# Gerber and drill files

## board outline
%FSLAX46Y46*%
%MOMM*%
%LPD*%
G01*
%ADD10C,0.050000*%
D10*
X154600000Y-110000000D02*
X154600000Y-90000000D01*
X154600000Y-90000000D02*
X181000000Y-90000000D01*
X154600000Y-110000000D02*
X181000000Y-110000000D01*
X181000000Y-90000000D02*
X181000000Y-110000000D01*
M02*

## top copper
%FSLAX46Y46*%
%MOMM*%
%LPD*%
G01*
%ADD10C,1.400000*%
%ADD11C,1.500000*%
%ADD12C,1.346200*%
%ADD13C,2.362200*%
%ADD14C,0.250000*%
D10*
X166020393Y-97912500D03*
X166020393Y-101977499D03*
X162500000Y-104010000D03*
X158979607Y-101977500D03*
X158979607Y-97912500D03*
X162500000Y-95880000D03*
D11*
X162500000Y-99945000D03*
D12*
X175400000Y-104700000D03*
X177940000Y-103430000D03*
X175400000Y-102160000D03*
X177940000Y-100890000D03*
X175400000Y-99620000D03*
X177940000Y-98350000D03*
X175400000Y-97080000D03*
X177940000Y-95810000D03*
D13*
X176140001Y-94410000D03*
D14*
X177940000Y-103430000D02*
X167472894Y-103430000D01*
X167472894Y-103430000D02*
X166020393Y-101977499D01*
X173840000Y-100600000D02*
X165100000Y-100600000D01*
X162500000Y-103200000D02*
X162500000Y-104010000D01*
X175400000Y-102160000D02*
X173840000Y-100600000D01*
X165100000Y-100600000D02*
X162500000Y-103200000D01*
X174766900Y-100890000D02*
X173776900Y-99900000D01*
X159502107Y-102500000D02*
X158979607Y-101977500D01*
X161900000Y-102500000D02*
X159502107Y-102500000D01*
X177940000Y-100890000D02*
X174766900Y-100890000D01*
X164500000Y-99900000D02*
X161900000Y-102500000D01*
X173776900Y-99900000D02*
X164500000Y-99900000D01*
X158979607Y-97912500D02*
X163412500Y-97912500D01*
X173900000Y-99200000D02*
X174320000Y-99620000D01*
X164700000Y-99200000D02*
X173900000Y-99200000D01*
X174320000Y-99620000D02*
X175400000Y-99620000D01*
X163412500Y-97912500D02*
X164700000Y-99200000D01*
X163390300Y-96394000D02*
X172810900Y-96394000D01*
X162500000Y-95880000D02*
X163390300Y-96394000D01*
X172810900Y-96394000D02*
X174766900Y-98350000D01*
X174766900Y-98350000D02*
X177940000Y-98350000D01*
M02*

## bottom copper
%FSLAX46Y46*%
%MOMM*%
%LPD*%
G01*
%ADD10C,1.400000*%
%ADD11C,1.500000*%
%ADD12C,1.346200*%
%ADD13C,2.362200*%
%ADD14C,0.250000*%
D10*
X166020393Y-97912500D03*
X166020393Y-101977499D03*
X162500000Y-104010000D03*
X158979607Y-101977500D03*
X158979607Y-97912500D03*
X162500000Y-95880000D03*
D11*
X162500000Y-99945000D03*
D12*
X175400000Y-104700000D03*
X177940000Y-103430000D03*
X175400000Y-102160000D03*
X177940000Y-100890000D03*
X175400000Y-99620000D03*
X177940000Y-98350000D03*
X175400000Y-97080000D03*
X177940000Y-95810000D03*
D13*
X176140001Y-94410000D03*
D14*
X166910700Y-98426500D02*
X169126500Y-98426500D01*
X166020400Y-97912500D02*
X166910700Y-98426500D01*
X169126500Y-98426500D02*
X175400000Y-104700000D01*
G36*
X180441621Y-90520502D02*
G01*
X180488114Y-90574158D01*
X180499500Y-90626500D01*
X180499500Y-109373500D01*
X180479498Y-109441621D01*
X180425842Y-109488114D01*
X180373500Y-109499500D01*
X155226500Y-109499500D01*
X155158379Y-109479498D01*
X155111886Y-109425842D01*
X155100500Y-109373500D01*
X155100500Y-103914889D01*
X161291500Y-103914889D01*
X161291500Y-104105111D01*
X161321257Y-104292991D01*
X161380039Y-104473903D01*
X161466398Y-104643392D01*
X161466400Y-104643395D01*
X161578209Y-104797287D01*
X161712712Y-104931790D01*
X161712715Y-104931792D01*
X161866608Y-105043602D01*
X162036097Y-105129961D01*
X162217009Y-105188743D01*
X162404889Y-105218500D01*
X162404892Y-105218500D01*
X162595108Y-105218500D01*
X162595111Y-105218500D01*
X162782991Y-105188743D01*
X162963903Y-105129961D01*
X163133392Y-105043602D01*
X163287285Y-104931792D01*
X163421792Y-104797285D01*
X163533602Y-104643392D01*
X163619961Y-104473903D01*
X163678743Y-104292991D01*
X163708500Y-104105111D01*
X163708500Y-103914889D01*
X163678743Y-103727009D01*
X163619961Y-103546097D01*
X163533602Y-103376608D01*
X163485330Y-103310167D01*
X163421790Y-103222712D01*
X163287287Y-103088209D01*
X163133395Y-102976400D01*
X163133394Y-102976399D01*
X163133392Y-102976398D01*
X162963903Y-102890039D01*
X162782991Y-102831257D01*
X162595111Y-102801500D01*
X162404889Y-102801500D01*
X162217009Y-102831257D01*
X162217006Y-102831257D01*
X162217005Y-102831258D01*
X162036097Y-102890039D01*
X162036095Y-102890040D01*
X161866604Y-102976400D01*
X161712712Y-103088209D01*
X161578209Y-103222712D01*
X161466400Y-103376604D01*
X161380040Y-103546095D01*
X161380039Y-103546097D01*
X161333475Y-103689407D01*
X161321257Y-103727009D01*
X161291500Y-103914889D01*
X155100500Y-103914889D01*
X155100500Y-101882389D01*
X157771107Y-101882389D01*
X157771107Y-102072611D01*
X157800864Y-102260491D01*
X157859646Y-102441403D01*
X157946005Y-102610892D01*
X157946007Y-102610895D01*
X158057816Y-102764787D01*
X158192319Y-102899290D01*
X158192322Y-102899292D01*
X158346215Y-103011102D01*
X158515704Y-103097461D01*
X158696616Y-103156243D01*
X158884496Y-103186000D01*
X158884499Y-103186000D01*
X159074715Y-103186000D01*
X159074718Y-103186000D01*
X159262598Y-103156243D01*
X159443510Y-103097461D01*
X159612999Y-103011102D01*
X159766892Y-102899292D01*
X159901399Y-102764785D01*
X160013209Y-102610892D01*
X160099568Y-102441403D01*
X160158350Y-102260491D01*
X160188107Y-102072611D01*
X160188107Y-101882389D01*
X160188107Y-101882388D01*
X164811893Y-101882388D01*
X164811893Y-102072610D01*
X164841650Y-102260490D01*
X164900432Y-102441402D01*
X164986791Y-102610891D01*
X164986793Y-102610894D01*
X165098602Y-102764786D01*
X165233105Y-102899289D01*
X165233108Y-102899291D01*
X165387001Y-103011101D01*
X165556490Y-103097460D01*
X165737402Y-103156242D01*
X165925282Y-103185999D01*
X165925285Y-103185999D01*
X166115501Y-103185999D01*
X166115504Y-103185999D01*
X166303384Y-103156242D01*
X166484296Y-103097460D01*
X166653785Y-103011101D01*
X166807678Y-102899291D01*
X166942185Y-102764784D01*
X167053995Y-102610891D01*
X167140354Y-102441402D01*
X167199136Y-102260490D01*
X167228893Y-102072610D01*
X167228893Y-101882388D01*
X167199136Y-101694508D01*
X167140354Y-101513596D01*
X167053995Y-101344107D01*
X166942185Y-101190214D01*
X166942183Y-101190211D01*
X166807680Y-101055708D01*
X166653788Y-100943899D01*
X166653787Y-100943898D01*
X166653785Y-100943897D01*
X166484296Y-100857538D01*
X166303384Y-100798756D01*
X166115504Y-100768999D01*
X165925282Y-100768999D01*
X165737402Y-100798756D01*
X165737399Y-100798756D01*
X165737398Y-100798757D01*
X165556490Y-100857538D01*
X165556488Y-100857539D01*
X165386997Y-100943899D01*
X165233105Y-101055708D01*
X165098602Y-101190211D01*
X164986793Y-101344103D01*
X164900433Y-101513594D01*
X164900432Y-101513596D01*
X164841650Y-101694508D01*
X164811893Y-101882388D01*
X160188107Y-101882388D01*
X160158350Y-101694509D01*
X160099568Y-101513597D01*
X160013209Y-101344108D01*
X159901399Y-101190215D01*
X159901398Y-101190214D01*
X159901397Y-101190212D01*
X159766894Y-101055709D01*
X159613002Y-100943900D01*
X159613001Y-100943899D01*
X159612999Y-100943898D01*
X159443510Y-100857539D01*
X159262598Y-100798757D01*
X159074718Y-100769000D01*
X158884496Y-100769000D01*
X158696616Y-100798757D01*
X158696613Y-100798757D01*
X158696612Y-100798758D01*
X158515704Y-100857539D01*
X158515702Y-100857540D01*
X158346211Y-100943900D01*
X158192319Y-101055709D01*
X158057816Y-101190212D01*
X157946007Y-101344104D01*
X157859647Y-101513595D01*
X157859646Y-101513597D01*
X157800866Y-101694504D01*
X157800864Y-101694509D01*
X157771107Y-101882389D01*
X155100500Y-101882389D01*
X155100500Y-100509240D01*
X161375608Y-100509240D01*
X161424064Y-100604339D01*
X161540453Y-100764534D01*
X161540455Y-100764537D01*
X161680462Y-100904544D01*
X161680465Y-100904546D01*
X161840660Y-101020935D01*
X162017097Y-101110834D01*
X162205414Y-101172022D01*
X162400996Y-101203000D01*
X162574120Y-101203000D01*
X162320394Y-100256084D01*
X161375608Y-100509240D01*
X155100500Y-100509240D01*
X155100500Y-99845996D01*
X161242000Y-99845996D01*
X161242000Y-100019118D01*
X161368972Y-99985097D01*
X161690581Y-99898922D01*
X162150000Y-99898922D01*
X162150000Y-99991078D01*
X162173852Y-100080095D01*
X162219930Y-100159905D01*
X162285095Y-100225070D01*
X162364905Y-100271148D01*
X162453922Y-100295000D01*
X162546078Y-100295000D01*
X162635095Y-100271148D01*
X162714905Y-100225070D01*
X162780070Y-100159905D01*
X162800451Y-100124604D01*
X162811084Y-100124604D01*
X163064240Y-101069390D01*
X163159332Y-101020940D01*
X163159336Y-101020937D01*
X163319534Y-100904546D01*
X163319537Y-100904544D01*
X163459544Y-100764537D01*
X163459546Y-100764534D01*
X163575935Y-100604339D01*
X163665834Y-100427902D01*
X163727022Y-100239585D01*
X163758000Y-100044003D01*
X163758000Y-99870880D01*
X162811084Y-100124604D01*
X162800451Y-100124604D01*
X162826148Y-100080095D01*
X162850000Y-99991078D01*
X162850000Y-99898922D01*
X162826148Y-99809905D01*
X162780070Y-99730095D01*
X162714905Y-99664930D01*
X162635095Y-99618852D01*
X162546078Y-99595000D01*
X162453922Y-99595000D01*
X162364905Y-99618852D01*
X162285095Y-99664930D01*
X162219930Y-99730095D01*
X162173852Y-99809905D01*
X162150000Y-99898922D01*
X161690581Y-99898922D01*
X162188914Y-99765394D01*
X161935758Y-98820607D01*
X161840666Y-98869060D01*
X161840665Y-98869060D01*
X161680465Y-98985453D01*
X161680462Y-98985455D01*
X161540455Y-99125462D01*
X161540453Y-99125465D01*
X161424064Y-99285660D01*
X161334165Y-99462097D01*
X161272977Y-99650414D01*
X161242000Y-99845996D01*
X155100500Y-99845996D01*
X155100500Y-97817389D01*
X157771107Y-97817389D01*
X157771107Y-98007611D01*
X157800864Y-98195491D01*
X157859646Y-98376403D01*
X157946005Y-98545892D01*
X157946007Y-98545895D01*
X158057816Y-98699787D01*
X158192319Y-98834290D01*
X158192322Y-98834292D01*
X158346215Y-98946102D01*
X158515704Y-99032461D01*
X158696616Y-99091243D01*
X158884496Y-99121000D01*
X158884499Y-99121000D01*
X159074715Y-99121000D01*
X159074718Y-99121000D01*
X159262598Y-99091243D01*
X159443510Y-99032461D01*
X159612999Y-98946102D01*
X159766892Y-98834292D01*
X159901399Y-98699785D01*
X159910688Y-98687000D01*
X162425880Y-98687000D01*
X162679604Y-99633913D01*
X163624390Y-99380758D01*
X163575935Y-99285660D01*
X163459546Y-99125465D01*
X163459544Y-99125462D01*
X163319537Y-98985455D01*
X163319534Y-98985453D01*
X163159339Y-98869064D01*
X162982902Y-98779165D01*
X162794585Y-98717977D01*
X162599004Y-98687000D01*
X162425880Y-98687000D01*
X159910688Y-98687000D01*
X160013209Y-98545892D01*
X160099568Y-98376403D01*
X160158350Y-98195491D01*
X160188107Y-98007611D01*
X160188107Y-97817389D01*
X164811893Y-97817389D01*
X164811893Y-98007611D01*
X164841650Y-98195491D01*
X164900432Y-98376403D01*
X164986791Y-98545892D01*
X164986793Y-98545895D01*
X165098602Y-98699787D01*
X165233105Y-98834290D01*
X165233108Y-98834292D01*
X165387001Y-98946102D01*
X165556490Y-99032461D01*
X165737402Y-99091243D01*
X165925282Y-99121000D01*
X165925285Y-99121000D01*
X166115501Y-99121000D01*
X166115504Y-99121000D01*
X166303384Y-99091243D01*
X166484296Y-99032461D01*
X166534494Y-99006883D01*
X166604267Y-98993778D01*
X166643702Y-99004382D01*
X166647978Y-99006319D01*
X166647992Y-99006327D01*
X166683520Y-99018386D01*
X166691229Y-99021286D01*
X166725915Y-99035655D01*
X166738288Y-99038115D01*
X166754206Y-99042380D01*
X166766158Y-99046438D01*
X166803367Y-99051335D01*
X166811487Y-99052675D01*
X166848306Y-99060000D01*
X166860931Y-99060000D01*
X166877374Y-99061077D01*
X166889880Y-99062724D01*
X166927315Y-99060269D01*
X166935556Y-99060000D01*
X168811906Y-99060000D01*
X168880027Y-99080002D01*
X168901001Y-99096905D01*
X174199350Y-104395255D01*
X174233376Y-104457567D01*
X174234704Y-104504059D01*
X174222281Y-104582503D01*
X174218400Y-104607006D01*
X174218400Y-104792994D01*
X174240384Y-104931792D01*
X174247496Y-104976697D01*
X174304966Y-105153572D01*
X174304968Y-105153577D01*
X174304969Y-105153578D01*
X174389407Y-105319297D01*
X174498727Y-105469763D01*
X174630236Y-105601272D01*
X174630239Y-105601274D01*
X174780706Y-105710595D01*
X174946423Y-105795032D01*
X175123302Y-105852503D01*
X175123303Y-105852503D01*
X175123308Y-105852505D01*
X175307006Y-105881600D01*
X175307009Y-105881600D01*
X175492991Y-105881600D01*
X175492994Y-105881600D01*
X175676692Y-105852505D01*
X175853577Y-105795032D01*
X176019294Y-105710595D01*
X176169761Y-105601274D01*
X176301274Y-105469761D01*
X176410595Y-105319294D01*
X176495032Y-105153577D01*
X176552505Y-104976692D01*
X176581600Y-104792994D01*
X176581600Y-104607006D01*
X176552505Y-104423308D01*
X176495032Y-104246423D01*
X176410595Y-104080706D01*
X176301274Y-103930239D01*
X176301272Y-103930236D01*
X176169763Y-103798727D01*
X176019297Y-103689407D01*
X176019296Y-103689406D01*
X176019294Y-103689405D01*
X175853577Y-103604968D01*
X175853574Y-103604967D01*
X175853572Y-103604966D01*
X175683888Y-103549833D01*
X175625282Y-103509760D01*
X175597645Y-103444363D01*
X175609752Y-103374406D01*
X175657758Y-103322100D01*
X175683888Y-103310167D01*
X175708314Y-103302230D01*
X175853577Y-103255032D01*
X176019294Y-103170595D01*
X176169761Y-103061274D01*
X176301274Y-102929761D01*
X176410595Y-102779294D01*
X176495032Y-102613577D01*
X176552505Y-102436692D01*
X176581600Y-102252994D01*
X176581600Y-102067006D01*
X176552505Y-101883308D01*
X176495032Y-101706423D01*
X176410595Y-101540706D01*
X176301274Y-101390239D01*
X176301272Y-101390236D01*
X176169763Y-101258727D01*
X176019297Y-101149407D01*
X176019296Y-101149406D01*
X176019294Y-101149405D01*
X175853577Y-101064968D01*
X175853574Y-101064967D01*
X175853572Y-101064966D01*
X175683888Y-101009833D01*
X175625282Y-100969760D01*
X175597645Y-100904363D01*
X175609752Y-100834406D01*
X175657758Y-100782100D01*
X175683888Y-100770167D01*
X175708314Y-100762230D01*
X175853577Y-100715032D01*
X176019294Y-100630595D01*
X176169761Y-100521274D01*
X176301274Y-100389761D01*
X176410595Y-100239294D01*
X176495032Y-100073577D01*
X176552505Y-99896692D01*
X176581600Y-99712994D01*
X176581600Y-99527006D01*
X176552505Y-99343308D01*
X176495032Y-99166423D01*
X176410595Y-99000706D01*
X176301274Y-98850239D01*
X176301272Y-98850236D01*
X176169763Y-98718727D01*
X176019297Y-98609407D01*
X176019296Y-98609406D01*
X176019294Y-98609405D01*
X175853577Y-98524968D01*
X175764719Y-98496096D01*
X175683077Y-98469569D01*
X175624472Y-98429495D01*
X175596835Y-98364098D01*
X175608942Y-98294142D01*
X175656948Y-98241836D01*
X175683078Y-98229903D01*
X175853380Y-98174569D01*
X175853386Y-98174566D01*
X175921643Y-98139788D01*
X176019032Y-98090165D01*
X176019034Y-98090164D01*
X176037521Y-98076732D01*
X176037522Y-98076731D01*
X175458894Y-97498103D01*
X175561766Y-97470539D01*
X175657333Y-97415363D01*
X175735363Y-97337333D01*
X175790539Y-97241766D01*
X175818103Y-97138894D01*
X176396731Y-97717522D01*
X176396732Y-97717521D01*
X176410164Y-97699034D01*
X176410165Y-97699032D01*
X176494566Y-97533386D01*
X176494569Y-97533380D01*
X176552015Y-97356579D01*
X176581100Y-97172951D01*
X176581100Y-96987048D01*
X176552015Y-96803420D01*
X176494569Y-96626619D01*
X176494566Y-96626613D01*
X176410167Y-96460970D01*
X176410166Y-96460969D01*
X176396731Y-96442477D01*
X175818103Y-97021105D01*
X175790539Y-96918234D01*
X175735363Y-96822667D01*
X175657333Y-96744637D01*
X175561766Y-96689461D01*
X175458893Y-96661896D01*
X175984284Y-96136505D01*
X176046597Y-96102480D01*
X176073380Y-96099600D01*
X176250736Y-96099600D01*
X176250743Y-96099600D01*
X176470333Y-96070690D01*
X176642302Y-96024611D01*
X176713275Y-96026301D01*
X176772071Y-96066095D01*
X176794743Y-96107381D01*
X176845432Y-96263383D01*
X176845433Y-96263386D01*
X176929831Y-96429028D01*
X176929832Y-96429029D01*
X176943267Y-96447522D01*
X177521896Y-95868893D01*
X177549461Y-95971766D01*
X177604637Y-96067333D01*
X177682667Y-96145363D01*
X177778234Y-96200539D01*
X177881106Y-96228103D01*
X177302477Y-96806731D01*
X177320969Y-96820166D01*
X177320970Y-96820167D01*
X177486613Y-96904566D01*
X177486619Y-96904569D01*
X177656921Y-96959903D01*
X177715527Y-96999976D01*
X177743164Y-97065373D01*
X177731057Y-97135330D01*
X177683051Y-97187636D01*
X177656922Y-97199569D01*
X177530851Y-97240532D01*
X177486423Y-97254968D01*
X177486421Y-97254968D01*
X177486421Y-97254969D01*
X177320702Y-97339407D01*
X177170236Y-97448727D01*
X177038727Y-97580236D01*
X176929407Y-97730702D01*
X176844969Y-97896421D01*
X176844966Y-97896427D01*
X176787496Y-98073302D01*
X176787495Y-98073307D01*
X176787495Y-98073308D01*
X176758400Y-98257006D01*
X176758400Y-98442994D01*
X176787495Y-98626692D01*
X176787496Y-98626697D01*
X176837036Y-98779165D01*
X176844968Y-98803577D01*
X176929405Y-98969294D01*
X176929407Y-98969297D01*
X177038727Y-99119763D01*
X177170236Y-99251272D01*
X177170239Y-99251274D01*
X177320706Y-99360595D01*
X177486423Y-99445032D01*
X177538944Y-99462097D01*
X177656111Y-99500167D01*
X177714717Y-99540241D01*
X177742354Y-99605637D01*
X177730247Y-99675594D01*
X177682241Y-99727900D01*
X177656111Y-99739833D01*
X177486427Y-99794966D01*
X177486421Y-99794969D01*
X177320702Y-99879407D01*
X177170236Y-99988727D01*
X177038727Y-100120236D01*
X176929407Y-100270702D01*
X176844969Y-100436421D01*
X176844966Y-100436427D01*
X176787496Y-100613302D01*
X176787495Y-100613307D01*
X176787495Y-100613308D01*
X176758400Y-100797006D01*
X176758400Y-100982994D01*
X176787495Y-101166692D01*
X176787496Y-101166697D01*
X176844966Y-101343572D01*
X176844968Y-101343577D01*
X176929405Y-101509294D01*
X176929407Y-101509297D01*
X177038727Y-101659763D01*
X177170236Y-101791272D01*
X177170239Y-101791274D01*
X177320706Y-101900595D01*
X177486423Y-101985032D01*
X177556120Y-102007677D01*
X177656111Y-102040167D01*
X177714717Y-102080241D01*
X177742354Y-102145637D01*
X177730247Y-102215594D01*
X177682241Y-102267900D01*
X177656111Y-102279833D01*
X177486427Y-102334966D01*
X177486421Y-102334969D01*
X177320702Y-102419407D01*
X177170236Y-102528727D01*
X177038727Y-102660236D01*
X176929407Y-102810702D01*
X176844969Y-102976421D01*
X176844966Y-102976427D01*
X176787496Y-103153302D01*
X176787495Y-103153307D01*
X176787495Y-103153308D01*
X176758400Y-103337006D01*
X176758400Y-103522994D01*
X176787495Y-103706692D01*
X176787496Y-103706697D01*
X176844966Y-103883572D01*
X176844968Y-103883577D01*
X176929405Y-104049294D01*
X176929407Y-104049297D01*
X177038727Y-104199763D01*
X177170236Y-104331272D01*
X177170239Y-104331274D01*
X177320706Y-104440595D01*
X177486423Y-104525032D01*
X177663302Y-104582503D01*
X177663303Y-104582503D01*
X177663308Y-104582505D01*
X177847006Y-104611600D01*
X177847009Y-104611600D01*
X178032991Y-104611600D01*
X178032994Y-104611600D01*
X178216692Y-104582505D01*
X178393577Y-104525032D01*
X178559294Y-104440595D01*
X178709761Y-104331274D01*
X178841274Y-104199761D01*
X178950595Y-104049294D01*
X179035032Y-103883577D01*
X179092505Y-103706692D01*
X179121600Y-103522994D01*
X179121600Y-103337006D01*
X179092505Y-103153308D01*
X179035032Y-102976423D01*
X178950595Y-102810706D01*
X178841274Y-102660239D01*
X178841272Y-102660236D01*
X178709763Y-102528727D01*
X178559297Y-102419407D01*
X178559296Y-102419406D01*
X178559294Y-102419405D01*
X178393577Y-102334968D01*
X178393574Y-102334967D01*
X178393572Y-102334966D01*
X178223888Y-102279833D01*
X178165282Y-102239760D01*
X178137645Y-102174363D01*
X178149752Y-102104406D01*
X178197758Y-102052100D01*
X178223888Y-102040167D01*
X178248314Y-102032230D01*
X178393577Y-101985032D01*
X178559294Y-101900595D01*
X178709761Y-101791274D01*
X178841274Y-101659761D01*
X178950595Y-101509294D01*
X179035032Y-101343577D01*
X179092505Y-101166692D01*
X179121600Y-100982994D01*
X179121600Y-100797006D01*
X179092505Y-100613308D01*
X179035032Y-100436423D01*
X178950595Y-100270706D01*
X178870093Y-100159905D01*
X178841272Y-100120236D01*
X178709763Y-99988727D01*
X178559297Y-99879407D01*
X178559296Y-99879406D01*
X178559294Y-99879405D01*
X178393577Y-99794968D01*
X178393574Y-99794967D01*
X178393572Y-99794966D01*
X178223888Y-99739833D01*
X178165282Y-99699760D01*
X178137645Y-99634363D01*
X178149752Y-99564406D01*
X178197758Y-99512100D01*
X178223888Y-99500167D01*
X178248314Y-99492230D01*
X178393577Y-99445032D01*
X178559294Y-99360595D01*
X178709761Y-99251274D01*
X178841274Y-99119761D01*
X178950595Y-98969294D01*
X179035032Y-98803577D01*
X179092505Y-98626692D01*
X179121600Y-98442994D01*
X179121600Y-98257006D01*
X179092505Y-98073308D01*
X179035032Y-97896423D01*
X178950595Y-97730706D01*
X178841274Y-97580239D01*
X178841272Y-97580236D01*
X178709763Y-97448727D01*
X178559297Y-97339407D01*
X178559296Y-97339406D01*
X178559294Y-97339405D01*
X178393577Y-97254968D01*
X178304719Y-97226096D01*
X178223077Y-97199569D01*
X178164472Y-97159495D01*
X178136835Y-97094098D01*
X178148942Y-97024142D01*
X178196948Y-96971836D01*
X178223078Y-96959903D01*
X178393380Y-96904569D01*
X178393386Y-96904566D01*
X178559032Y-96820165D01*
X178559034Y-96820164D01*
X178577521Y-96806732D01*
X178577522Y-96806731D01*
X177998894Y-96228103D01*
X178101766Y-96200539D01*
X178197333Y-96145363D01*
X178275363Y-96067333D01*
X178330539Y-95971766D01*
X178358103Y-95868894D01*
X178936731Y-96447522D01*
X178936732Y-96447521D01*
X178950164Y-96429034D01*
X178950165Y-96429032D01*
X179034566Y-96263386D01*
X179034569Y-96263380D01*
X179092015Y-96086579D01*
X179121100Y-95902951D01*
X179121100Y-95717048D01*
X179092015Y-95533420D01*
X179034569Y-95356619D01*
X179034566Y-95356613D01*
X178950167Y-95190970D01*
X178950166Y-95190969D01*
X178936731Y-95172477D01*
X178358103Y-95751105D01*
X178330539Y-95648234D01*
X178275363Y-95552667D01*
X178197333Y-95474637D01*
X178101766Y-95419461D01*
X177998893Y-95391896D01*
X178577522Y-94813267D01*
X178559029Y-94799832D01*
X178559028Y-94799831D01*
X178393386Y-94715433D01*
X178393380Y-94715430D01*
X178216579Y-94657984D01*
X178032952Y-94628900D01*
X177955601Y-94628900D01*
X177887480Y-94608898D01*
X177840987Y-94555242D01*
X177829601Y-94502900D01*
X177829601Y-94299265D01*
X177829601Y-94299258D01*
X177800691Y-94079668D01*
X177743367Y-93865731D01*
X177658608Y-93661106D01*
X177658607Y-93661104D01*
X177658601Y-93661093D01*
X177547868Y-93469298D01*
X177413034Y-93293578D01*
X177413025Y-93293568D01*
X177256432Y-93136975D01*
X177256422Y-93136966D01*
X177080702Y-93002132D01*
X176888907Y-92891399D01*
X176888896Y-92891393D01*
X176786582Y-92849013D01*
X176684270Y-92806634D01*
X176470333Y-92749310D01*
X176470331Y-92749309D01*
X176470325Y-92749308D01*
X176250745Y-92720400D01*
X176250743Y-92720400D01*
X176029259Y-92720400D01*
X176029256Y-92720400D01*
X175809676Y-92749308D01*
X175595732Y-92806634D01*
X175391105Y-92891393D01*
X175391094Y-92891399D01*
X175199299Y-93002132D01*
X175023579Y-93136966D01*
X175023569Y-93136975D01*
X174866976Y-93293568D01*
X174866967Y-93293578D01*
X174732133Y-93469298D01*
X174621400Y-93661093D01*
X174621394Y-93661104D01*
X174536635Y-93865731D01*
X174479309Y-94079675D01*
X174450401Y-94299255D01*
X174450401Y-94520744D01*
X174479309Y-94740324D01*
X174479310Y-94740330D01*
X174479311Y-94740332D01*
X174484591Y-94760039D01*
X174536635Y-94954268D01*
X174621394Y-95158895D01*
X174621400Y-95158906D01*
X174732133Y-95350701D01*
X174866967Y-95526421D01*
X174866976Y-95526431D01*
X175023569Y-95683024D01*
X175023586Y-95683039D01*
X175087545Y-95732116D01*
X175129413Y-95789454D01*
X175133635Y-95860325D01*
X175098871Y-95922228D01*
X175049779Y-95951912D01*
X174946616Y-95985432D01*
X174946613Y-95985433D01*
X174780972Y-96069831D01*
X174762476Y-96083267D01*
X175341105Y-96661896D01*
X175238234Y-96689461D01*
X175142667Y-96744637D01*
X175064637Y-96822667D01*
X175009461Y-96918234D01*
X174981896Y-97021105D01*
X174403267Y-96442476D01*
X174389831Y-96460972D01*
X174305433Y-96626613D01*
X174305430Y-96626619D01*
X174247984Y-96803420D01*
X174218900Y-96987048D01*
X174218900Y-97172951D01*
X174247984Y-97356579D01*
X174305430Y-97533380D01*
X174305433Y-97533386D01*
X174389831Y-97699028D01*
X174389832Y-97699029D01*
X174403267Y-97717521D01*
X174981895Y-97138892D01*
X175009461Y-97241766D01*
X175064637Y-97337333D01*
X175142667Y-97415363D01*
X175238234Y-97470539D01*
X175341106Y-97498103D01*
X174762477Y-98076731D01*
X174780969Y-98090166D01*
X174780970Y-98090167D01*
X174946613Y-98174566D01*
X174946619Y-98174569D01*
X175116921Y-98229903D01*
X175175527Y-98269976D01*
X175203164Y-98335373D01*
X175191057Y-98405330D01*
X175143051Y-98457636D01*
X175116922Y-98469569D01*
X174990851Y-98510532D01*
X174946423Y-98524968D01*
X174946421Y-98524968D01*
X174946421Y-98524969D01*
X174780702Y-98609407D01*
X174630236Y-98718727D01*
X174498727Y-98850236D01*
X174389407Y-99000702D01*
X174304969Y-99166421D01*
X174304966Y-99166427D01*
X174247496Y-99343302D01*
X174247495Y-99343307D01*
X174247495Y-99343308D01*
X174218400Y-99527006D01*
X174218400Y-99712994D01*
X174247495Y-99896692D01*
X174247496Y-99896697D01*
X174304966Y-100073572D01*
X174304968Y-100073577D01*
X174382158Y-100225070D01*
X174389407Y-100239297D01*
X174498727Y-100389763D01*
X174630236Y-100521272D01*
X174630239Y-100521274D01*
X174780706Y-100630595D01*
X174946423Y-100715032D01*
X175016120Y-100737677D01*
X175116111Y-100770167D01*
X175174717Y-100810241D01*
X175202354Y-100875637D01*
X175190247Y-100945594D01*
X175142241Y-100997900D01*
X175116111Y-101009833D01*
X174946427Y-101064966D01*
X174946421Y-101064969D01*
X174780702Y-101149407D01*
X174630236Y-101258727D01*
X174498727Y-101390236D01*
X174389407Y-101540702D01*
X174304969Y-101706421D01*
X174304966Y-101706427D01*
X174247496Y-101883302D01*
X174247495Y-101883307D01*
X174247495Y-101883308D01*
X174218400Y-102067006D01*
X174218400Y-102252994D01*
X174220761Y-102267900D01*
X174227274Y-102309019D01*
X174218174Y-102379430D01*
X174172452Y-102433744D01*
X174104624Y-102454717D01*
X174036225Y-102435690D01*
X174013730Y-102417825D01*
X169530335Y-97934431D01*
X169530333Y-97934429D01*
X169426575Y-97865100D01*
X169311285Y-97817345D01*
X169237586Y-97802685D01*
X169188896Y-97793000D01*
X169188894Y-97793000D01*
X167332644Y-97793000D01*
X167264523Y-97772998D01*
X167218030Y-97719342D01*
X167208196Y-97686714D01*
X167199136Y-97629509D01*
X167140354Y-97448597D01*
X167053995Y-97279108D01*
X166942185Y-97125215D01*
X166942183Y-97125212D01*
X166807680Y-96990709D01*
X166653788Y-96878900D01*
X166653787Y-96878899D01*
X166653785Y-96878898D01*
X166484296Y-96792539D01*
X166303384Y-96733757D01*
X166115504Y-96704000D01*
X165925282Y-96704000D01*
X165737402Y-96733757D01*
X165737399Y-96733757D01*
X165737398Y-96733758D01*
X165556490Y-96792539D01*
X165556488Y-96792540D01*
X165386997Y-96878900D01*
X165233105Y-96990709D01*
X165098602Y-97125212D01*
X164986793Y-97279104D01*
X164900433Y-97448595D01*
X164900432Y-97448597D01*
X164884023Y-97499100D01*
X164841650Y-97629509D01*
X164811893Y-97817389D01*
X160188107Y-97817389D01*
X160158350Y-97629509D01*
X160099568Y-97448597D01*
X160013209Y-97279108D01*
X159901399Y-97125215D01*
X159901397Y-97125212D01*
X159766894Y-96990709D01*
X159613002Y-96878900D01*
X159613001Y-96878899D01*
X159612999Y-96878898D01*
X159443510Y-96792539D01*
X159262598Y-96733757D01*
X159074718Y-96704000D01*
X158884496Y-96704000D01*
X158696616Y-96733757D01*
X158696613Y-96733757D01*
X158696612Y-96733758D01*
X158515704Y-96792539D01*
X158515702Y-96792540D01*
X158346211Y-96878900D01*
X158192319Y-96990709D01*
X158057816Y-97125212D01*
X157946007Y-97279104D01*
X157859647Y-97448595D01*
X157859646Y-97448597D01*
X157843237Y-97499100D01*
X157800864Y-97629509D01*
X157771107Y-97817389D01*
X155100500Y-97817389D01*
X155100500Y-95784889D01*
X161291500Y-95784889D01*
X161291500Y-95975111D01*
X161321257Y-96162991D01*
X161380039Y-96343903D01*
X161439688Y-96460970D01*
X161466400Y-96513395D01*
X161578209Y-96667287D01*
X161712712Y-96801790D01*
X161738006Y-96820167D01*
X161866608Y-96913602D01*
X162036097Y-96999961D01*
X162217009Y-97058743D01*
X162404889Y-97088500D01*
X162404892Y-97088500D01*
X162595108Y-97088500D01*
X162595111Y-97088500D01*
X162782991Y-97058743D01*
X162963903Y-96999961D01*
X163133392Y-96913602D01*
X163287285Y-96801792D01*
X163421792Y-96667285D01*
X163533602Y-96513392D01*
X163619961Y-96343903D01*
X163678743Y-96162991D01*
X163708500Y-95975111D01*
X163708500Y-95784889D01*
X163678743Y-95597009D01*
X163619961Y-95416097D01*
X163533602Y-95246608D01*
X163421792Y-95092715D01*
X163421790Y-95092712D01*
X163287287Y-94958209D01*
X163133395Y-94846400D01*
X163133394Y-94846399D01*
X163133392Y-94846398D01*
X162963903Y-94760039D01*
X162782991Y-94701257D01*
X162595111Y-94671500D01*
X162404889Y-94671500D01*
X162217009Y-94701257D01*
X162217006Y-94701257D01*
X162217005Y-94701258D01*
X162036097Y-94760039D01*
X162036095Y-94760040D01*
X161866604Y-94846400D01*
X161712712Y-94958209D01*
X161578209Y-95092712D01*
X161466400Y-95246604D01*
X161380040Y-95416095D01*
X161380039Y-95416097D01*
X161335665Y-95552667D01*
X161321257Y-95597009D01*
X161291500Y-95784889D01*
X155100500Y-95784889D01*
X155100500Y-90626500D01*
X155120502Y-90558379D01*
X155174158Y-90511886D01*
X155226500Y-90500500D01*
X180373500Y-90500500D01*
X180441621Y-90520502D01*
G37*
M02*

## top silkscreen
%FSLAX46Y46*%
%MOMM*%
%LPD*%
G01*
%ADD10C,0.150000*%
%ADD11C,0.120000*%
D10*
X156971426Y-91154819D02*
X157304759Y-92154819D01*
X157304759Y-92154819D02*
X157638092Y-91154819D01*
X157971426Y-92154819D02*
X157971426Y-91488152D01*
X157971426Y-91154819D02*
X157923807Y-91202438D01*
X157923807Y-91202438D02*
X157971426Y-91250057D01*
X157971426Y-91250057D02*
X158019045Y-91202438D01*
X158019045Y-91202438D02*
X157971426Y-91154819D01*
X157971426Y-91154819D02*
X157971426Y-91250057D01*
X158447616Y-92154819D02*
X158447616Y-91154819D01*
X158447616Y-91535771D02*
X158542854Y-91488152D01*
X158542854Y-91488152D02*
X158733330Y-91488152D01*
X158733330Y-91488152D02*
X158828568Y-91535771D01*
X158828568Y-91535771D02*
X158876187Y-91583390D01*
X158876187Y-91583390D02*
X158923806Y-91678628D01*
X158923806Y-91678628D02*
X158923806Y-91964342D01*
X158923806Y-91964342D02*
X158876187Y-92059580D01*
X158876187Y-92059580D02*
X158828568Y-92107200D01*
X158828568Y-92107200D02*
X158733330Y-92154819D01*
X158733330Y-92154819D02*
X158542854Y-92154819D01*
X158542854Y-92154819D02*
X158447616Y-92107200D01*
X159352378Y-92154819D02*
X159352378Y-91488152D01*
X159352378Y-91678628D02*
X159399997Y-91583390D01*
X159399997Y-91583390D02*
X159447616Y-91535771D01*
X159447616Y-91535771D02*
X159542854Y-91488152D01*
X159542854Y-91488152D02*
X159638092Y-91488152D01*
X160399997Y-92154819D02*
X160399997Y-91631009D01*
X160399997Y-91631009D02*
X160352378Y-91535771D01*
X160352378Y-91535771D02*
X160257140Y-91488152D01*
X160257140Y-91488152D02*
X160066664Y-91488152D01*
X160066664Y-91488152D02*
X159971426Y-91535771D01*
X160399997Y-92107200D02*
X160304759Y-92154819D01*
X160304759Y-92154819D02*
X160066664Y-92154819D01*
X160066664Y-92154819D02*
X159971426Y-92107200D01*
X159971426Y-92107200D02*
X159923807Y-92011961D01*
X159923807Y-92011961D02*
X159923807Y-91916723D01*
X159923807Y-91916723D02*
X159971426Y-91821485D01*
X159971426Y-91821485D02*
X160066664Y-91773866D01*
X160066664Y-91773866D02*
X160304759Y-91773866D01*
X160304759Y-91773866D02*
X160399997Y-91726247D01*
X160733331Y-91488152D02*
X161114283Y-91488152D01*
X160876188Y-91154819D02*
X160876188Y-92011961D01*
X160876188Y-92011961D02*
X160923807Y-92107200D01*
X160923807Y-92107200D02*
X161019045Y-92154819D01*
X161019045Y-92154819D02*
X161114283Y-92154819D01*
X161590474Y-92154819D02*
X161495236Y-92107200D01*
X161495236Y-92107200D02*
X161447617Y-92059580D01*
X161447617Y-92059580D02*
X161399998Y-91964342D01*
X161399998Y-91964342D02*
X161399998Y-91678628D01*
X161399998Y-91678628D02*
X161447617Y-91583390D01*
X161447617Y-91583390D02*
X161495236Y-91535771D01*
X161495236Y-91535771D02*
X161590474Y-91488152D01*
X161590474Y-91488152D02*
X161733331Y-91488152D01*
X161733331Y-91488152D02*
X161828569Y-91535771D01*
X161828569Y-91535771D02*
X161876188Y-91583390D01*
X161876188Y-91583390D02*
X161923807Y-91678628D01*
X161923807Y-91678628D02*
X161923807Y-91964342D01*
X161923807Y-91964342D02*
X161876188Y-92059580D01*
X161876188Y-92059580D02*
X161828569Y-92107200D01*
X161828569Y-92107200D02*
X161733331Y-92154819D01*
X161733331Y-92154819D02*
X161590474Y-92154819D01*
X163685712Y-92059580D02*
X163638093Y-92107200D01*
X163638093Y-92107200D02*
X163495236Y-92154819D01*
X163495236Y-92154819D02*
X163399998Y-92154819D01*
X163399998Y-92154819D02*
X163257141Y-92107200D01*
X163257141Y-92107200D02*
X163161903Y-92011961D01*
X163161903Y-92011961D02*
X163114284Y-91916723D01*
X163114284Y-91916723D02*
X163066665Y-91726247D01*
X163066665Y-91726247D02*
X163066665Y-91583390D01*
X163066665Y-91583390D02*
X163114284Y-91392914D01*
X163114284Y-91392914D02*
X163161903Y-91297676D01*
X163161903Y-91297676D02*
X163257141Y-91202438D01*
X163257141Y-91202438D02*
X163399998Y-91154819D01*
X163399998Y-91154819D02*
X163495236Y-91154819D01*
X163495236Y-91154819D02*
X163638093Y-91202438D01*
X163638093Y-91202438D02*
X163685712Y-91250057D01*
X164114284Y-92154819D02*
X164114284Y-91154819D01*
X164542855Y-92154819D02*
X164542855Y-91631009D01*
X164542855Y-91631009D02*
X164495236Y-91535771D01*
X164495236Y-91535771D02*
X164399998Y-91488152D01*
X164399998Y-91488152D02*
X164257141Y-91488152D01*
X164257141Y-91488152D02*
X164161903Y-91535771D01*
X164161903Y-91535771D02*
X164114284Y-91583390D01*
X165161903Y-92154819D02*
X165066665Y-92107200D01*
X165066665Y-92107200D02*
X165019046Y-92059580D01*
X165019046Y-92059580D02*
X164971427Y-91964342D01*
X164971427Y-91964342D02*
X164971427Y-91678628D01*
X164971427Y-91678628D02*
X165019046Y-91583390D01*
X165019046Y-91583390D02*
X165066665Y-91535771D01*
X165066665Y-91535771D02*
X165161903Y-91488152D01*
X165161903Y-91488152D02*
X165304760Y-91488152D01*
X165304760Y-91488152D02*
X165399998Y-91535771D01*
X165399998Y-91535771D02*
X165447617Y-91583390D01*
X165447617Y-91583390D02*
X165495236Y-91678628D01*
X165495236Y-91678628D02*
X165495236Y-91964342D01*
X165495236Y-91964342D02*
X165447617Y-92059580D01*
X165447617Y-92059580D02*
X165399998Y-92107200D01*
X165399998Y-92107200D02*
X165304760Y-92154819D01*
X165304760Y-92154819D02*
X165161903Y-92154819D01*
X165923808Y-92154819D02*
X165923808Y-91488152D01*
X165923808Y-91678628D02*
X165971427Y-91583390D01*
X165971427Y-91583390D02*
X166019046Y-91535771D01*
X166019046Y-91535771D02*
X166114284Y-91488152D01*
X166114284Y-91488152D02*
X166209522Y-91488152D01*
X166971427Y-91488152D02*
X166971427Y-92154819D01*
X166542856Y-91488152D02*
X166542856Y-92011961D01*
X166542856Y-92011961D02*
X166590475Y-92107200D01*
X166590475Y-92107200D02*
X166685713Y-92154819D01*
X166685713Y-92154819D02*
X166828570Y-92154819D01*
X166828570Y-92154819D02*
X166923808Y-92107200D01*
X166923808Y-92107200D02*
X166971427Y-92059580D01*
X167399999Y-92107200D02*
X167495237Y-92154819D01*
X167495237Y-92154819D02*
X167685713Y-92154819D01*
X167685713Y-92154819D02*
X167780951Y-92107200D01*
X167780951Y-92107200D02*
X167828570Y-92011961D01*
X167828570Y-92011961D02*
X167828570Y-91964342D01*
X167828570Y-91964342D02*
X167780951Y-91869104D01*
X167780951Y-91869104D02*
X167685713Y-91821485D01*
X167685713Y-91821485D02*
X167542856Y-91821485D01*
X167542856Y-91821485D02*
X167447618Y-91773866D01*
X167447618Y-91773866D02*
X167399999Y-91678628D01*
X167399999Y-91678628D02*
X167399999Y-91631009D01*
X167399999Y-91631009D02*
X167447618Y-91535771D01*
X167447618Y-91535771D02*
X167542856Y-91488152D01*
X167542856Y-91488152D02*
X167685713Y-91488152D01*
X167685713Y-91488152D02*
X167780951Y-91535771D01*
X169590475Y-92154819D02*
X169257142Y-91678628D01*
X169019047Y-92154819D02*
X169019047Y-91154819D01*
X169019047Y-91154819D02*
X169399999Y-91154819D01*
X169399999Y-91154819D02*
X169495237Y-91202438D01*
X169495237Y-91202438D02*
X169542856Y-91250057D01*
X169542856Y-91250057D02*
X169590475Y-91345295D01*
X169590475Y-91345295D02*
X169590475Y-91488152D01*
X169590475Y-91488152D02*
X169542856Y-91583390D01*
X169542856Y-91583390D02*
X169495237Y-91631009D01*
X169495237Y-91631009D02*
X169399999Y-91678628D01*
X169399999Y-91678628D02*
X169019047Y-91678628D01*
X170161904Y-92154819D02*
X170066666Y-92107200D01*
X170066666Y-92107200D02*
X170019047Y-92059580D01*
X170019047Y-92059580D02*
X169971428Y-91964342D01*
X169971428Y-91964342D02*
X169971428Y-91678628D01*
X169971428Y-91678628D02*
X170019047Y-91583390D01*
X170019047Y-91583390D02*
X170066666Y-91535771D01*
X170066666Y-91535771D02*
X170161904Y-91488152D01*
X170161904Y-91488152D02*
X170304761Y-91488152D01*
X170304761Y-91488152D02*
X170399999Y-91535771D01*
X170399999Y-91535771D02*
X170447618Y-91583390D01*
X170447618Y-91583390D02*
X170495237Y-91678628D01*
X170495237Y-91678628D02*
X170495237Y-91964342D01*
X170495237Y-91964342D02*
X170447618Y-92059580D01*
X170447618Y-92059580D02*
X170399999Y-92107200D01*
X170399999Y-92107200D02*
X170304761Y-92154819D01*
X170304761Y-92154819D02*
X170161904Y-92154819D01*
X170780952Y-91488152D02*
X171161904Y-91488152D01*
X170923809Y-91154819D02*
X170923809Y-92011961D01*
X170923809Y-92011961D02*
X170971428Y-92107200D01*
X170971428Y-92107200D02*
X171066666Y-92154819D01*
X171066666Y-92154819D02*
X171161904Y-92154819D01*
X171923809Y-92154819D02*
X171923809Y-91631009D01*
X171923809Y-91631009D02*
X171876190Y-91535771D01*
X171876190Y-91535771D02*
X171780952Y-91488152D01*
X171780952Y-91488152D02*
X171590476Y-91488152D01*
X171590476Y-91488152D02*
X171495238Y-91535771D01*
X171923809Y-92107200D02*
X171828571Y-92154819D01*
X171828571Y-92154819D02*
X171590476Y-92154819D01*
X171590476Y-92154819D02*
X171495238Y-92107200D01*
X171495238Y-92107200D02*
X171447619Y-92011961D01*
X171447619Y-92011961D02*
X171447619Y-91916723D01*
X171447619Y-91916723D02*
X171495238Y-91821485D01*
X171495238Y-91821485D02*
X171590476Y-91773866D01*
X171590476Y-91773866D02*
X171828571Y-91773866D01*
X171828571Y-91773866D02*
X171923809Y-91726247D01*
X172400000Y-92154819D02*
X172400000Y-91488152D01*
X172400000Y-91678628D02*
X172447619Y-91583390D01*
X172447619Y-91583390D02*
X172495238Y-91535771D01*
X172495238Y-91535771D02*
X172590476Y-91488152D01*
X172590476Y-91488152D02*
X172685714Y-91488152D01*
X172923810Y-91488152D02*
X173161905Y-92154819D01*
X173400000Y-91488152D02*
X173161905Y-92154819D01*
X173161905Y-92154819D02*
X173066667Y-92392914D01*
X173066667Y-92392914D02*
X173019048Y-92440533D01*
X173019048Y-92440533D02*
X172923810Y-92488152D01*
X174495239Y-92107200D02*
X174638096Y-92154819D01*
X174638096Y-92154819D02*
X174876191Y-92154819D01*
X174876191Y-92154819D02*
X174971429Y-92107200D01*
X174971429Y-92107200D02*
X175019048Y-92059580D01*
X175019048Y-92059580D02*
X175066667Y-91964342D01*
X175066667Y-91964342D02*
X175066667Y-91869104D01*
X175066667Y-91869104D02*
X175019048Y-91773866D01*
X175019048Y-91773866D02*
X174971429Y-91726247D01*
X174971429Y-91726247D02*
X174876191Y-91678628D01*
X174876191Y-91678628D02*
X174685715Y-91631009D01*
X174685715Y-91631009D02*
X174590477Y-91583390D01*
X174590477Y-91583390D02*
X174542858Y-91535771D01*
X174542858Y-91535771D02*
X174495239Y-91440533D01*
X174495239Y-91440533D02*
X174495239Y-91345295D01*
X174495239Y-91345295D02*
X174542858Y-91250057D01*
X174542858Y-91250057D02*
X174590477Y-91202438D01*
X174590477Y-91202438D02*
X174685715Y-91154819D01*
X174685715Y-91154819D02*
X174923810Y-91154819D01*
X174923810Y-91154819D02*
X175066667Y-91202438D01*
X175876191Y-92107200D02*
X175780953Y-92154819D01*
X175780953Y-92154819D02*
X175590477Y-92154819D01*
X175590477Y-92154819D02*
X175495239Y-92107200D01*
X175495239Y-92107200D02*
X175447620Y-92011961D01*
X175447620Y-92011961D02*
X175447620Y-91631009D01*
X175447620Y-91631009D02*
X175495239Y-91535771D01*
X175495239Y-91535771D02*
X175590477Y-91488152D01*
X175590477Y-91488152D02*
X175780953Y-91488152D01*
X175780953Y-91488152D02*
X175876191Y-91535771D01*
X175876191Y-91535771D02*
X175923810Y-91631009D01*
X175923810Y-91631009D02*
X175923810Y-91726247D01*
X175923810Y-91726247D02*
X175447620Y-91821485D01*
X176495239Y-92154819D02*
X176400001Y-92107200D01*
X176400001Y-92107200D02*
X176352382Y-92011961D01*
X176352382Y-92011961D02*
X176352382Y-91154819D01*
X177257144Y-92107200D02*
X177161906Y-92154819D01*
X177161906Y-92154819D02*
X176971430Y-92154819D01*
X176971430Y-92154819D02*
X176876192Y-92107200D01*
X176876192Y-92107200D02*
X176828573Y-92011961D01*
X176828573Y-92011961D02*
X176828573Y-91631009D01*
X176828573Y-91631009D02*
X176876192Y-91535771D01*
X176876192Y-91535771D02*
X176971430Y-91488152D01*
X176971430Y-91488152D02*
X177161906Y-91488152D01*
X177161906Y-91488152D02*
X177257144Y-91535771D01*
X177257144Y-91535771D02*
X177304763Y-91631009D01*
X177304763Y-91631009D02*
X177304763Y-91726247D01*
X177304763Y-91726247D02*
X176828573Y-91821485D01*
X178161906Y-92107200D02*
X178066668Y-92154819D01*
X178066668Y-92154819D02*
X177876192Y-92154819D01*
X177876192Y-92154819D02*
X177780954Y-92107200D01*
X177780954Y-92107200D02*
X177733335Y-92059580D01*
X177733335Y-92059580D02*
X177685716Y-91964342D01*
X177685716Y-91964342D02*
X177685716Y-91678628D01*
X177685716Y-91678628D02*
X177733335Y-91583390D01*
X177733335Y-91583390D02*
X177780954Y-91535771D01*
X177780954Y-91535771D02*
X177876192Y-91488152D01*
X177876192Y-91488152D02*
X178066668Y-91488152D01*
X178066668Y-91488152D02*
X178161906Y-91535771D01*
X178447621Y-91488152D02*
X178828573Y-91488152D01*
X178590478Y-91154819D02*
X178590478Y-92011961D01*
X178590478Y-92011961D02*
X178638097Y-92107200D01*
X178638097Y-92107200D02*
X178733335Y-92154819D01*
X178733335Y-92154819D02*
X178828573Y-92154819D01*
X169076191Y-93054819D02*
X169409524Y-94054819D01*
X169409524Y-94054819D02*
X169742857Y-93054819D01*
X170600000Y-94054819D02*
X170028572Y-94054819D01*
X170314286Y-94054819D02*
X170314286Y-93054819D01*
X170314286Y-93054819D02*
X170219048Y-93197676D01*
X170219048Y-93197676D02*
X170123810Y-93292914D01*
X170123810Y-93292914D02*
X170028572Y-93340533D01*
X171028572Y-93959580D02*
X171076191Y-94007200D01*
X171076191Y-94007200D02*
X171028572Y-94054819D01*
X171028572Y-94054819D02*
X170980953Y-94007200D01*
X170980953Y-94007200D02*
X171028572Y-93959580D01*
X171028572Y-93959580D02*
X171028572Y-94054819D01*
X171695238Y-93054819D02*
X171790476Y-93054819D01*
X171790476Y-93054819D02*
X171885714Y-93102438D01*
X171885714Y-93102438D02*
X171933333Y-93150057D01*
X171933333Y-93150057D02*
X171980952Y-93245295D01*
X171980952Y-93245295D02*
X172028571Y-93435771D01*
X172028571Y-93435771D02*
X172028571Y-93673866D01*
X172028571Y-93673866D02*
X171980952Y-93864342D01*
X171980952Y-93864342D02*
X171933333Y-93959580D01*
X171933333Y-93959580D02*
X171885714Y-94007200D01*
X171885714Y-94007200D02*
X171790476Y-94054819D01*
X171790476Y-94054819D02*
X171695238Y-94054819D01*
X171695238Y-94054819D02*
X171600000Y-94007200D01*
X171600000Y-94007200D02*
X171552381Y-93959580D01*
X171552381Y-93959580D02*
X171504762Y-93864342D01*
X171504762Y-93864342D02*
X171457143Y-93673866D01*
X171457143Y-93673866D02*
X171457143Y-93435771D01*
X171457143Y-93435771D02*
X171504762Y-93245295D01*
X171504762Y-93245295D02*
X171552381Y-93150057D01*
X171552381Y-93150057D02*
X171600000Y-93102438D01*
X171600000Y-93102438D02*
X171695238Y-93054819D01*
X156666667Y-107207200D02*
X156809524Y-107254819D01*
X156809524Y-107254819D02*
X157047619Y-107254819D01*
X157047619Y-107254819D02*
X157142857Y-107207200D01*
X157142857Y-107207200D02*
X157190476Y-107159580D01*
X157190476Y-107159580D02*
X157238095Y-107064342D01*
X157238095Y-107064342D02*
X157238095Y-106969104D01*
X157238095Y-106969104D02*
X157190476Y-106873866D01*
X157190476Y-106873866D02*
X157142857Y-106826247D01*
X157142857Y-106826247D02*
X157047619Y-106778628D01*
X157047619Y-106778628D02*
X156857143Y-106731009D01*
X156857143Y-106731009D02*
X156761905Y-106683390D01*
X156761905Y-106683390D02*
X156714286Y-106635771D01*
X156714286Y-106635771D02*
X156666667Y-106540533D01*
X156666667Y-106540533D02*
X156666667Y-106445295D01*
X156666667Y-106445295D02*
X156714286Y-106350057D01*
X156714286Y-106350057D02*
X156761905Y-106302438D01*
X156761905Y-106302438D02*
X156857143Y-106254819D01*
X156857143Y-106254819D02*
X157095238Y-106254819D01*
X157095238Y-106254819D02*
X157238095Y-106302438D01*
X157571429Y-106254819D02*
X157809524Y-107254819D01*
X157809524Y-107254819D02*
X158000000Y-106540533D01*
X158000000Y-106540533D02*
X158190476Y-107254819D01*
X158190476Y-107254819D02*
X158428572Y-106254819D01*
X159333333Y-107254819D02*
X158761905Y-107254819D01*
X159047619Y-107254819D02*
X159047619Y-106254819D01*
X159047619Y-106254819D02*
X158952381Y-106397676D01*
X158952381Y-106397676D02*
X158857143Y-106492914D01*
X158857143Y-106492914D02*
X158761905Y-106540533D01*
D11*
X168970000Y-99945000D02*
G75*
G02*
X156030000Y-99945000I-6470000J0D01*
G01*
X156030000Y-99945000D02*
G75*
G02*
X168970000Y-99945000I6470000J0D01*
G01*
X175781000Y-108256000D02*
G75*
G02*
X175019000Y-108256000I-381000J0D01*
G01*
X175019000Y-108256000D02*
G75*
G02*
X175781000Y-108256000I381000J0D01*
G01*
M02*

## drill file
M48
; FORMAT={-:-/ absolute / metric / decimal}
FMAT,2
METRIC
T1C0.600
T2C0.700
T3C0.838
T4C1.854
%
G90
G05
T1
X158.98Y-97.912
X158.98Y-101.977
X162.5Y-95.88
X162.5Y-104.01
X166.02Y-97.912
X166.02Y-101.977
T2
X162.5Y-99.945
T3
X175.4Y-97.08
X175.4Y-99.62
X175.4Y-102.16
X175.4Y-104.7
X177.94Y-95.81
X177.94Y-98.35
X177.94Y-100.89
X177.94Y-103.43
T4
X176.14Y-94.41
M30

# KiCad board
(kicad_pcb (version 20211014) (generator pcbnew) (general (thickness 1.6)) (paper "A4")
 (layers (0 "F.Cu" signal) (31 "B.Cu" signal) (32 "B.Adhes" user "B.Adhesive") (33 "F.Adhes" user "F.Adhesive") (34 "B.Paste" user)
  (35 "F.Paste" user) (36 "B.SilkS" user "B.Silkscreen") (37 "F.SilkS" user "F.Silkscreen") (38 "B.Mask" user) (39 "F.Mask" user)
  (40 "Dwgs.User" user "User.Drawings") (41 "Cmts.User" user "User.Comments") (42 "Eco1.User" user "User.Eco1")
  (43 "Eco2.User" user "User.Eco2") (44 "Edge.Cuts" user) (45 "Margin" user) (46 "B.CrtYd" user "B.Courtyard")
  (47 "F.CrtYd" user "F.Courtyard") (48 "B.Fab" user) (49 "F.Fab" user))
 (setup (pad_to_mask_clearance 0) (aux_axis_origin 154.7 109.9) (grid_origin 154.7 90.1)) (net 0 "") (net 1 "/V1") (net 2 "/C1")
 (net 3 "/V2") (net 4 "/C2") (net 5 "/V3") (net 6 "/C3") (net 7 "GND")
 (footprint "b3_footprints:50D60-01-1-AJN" (layer "F.Cu") (at 162.5 99.945)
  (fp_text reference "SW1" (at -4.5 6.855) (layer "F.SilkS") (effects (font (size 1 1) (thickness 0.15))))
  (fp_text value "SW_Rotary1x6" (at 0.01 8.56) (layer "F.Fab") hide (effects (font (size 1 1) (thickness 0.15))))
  (fp_circle (center 0 0) (end 0 6.47) (layer "F.SilkS") (width 0.12) (fill none))
  (pad "1" thru_hole circle (at 3.520393 -2.0325 60) (size 1.4 1.4) (drill 0.6) (layers *.Cu *.Mask) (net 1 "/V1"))
  (pad "2" thru_hole circle (at 3.520393 2.032499 60) (size 1.4 1.4) (drill 0.6) (layers *.Cu *.Mask) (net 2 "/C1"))
  (pad "3" thru_hole circle (at 0 4.065 60) (size 1.4 1.4) (drill 0.6) (layers *.Cu *.Mask) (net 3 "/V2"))
  (pad "4" thru_hole circle (at -3.520393 2.0325 60) (size 1.4 1.4) (drill 0.6) (layers *.Cu *.Mask) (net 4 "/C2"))
  (pad "5" thru_hole circle (at -3.520393 -2.0325 60) (size 1.4 1.4) (drill 0.6) (layers *.Cu *.Mask) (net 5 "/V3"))
  (pad "6" thru_hole circle (at 0 -4.065 60) (size 1.4 1.4) (drill 0.6) (layers *.Cu *.Mask) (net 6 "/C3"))
  (pad "7" thru_hole circle (at 0 0 60) (size 1.5 1.5) (drill 0.7) (layers *.Cu *.Mask) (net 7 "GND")))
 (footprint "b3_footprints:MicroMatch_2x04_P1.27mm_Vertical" (layer "B.Cu") (at 175.4 104.7 90)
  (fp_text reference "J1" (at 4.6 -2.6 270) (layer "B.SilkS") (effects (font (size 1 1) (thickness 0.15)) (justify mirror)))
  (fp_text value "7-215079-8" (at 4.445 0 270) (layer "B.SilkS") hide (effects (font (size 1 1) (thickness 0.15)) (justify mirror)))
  (fp_circle (center -3.556 0) (end -3.175 0) (layer "F.SilkS") (width 0.12) (fill none))
  (pad "1" thru_hole circle locked (at 0 0 90) (size 1.3462 1.3462) (drill 0.8382) (layers *.Cu *.Mask) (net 1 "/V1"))
  (pad "2" thru_hole circle locked (at 1.27 2.54 90) (size 1.3462 1.3462) (drill 0.8382) (layers *.Cu *.Mask) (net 2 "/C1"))
  (pad "3" thru_hole circle locked (at 2.54 0 90) (size 1.3462 1.3462) (drill 0.8382) (layers *.Cu *.Mask) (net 3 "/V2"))
  (pad "4" thru_hole circle locked (at 3.81 2.54 90) (size 1.3462 1.3462) (drill 0.8382) (layers *.Cu *.Mask) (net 4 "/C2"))
  (pad "5" thru_hole circle locked (at 5.08 0 90) (size 1.3462 1.3462) (drill 0.8382) (layers *.Cu *.Mask) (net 5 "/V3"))
  (pad "6" thru_hole circle locked (at 6.35 2.54 90) (size 1.3462 1.3462) (drill 0.8382) (layers *.Cu *.Mask) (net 6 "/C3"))
  (pad "7" thru_hole circle locked (at 7.62 0 90) (size 1.3462 1.3462) (drill 0.8382) (layers *.Cu *.Mask) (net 7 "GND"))
  (pad "8" thru_hole circle locked (at 8.89 2.54 90) (size 1.3462 1.3462) (drill 0.8382) (layers *.Cu *.Mask) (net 7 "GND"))
  (pad "9" thru_hole circle locked (at 10.29 0.740001 90) (size 2.3622 2.3622) (drill 1.8542) (layers *.Cu *.Mask)))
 (gr_line (start 154.6 110) (end 154.6 90) (layer "Edge.Cuts") (width 0.05))
 (gr_line (start 154.6 90) (end 181 90) (layer "Edge.Cuts") (width 0.05))
 (gr_line (start 154.6 110) (end 181 110) (layer "Edge.Cuts") (width 0.05))
 (gr_line (start 181 90) (end 181 110) (layer "Edge.Cuts") (width 0.05))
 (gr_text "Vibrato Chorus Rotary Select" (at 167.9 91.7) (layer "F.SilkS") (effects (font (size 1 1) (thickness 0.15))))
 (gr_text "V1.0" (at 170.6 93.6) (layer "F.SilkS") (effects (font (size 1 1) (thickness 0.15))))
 (segment (start 166.9107 98.4265) (end 169.1265 98.4265) (width 0.25) (layer "B.Cu") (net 1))
 (segment (start 166.0204 97.9125) (end 166.9107 98.4265) (width 0.25) (layer "B.Cu") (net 1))
 (segment (start 169.1265 98.4265) (end 175.4 104.7) (width 0.25) (layer "B.Cu") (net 1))
 (segment (start 177.94 103.43) (end 167.472894 103.43) (width 0.25) (layer "F.Cu") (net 2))
 (segment (start 167.472894 103.43) (end 166.020393 101.977499) (width 0.25) (layer "F.Cu") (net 2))
 (segment (start 173.84 100.6) (end 165.1 100.6) (width 0.25) (layer "F.Cu") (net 3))
 (segment (start 162.5 103.2) (end 162.5 104.01) (width 0.25) (layer "F.Cu") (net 3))
 (segment (start 175.4 102.16) (end 173.84 100.6) (width 0.25) (layer "F.Cu") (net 3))
 (segment (start 165.1 100.6) (end 162.5 103.2) (width 0.25) (layer "F.Cu") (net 3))
 (segment (start 174.7669 100.89) (end 173.7769 99.9) (width 0.25) (layer "F.Cu") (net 4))
 (segment (start 159.502107 102.5) (end 158.979607 101.9775) (width 0.25) (layer "F.Cu") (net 4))
 (segment (start 161.9 102.5) (end 159.502107 102.5) (width 0.25) (layer "F.Cu") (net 4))
 (segment (start 177.94 100.89) (end 174.7669 100.89) (width 0.25) (layer "F.Cu") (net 4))
 (segment (start 164.5 99.9) (end 161.9 102.5) (width 0.25) (layer "F.Cu") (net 4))
 (segment (start 173.7769 99.9) (end 164.5 99.9) (width 0.25) (layer "F.Cu") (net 4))
 (segment (start 158.979607 97.9125) (end 163.4125 97.9125) (width 0.25) (layer "F.Cu") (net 5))
 (segment (start 173.9 99.2) (end 174.32 99.62) (width 0.25) (layer "F.Cu") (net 5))
 (segment (start 164.7 99.2) (end 173.9 99.2) (width 0.25) (layer "F.Cu") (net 5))
 (segment (start 174.32 99.62) (end 175.4 99.62) (width 0.25) (layer "F.Cu") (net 5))
 (segment (start 163.4125 97.9125) (end 164.7 99.2) (width 0.25) (layer "F.Cu") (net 5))
 (segment (start 163.3903 96.394) (end 172.8109 96.394) (width 0.25) (layer "F.Cu") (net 6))
 (segment (start 162.5 95.88) (end 163.3903 96.394) (width 0.25) (layer "F.Cu") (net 6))
 (segment (start 172.8109 96.394) (end 174.7669 98.35) (width 0.25) (layer "F.Cu") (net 6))
 (segment (start 174.7669 98.35) (end 177.94 98.35) (width 0.25) (layer "F.Cu") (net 6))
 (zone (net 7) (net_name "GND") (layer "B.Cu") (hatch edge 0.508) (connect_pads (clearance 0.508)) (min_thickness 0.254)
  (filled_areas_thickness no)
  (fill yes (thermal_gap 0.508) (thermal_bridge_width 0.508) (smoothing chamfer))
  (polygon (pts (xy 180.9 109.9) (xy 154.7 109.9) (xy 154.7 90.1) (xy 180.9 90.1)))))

